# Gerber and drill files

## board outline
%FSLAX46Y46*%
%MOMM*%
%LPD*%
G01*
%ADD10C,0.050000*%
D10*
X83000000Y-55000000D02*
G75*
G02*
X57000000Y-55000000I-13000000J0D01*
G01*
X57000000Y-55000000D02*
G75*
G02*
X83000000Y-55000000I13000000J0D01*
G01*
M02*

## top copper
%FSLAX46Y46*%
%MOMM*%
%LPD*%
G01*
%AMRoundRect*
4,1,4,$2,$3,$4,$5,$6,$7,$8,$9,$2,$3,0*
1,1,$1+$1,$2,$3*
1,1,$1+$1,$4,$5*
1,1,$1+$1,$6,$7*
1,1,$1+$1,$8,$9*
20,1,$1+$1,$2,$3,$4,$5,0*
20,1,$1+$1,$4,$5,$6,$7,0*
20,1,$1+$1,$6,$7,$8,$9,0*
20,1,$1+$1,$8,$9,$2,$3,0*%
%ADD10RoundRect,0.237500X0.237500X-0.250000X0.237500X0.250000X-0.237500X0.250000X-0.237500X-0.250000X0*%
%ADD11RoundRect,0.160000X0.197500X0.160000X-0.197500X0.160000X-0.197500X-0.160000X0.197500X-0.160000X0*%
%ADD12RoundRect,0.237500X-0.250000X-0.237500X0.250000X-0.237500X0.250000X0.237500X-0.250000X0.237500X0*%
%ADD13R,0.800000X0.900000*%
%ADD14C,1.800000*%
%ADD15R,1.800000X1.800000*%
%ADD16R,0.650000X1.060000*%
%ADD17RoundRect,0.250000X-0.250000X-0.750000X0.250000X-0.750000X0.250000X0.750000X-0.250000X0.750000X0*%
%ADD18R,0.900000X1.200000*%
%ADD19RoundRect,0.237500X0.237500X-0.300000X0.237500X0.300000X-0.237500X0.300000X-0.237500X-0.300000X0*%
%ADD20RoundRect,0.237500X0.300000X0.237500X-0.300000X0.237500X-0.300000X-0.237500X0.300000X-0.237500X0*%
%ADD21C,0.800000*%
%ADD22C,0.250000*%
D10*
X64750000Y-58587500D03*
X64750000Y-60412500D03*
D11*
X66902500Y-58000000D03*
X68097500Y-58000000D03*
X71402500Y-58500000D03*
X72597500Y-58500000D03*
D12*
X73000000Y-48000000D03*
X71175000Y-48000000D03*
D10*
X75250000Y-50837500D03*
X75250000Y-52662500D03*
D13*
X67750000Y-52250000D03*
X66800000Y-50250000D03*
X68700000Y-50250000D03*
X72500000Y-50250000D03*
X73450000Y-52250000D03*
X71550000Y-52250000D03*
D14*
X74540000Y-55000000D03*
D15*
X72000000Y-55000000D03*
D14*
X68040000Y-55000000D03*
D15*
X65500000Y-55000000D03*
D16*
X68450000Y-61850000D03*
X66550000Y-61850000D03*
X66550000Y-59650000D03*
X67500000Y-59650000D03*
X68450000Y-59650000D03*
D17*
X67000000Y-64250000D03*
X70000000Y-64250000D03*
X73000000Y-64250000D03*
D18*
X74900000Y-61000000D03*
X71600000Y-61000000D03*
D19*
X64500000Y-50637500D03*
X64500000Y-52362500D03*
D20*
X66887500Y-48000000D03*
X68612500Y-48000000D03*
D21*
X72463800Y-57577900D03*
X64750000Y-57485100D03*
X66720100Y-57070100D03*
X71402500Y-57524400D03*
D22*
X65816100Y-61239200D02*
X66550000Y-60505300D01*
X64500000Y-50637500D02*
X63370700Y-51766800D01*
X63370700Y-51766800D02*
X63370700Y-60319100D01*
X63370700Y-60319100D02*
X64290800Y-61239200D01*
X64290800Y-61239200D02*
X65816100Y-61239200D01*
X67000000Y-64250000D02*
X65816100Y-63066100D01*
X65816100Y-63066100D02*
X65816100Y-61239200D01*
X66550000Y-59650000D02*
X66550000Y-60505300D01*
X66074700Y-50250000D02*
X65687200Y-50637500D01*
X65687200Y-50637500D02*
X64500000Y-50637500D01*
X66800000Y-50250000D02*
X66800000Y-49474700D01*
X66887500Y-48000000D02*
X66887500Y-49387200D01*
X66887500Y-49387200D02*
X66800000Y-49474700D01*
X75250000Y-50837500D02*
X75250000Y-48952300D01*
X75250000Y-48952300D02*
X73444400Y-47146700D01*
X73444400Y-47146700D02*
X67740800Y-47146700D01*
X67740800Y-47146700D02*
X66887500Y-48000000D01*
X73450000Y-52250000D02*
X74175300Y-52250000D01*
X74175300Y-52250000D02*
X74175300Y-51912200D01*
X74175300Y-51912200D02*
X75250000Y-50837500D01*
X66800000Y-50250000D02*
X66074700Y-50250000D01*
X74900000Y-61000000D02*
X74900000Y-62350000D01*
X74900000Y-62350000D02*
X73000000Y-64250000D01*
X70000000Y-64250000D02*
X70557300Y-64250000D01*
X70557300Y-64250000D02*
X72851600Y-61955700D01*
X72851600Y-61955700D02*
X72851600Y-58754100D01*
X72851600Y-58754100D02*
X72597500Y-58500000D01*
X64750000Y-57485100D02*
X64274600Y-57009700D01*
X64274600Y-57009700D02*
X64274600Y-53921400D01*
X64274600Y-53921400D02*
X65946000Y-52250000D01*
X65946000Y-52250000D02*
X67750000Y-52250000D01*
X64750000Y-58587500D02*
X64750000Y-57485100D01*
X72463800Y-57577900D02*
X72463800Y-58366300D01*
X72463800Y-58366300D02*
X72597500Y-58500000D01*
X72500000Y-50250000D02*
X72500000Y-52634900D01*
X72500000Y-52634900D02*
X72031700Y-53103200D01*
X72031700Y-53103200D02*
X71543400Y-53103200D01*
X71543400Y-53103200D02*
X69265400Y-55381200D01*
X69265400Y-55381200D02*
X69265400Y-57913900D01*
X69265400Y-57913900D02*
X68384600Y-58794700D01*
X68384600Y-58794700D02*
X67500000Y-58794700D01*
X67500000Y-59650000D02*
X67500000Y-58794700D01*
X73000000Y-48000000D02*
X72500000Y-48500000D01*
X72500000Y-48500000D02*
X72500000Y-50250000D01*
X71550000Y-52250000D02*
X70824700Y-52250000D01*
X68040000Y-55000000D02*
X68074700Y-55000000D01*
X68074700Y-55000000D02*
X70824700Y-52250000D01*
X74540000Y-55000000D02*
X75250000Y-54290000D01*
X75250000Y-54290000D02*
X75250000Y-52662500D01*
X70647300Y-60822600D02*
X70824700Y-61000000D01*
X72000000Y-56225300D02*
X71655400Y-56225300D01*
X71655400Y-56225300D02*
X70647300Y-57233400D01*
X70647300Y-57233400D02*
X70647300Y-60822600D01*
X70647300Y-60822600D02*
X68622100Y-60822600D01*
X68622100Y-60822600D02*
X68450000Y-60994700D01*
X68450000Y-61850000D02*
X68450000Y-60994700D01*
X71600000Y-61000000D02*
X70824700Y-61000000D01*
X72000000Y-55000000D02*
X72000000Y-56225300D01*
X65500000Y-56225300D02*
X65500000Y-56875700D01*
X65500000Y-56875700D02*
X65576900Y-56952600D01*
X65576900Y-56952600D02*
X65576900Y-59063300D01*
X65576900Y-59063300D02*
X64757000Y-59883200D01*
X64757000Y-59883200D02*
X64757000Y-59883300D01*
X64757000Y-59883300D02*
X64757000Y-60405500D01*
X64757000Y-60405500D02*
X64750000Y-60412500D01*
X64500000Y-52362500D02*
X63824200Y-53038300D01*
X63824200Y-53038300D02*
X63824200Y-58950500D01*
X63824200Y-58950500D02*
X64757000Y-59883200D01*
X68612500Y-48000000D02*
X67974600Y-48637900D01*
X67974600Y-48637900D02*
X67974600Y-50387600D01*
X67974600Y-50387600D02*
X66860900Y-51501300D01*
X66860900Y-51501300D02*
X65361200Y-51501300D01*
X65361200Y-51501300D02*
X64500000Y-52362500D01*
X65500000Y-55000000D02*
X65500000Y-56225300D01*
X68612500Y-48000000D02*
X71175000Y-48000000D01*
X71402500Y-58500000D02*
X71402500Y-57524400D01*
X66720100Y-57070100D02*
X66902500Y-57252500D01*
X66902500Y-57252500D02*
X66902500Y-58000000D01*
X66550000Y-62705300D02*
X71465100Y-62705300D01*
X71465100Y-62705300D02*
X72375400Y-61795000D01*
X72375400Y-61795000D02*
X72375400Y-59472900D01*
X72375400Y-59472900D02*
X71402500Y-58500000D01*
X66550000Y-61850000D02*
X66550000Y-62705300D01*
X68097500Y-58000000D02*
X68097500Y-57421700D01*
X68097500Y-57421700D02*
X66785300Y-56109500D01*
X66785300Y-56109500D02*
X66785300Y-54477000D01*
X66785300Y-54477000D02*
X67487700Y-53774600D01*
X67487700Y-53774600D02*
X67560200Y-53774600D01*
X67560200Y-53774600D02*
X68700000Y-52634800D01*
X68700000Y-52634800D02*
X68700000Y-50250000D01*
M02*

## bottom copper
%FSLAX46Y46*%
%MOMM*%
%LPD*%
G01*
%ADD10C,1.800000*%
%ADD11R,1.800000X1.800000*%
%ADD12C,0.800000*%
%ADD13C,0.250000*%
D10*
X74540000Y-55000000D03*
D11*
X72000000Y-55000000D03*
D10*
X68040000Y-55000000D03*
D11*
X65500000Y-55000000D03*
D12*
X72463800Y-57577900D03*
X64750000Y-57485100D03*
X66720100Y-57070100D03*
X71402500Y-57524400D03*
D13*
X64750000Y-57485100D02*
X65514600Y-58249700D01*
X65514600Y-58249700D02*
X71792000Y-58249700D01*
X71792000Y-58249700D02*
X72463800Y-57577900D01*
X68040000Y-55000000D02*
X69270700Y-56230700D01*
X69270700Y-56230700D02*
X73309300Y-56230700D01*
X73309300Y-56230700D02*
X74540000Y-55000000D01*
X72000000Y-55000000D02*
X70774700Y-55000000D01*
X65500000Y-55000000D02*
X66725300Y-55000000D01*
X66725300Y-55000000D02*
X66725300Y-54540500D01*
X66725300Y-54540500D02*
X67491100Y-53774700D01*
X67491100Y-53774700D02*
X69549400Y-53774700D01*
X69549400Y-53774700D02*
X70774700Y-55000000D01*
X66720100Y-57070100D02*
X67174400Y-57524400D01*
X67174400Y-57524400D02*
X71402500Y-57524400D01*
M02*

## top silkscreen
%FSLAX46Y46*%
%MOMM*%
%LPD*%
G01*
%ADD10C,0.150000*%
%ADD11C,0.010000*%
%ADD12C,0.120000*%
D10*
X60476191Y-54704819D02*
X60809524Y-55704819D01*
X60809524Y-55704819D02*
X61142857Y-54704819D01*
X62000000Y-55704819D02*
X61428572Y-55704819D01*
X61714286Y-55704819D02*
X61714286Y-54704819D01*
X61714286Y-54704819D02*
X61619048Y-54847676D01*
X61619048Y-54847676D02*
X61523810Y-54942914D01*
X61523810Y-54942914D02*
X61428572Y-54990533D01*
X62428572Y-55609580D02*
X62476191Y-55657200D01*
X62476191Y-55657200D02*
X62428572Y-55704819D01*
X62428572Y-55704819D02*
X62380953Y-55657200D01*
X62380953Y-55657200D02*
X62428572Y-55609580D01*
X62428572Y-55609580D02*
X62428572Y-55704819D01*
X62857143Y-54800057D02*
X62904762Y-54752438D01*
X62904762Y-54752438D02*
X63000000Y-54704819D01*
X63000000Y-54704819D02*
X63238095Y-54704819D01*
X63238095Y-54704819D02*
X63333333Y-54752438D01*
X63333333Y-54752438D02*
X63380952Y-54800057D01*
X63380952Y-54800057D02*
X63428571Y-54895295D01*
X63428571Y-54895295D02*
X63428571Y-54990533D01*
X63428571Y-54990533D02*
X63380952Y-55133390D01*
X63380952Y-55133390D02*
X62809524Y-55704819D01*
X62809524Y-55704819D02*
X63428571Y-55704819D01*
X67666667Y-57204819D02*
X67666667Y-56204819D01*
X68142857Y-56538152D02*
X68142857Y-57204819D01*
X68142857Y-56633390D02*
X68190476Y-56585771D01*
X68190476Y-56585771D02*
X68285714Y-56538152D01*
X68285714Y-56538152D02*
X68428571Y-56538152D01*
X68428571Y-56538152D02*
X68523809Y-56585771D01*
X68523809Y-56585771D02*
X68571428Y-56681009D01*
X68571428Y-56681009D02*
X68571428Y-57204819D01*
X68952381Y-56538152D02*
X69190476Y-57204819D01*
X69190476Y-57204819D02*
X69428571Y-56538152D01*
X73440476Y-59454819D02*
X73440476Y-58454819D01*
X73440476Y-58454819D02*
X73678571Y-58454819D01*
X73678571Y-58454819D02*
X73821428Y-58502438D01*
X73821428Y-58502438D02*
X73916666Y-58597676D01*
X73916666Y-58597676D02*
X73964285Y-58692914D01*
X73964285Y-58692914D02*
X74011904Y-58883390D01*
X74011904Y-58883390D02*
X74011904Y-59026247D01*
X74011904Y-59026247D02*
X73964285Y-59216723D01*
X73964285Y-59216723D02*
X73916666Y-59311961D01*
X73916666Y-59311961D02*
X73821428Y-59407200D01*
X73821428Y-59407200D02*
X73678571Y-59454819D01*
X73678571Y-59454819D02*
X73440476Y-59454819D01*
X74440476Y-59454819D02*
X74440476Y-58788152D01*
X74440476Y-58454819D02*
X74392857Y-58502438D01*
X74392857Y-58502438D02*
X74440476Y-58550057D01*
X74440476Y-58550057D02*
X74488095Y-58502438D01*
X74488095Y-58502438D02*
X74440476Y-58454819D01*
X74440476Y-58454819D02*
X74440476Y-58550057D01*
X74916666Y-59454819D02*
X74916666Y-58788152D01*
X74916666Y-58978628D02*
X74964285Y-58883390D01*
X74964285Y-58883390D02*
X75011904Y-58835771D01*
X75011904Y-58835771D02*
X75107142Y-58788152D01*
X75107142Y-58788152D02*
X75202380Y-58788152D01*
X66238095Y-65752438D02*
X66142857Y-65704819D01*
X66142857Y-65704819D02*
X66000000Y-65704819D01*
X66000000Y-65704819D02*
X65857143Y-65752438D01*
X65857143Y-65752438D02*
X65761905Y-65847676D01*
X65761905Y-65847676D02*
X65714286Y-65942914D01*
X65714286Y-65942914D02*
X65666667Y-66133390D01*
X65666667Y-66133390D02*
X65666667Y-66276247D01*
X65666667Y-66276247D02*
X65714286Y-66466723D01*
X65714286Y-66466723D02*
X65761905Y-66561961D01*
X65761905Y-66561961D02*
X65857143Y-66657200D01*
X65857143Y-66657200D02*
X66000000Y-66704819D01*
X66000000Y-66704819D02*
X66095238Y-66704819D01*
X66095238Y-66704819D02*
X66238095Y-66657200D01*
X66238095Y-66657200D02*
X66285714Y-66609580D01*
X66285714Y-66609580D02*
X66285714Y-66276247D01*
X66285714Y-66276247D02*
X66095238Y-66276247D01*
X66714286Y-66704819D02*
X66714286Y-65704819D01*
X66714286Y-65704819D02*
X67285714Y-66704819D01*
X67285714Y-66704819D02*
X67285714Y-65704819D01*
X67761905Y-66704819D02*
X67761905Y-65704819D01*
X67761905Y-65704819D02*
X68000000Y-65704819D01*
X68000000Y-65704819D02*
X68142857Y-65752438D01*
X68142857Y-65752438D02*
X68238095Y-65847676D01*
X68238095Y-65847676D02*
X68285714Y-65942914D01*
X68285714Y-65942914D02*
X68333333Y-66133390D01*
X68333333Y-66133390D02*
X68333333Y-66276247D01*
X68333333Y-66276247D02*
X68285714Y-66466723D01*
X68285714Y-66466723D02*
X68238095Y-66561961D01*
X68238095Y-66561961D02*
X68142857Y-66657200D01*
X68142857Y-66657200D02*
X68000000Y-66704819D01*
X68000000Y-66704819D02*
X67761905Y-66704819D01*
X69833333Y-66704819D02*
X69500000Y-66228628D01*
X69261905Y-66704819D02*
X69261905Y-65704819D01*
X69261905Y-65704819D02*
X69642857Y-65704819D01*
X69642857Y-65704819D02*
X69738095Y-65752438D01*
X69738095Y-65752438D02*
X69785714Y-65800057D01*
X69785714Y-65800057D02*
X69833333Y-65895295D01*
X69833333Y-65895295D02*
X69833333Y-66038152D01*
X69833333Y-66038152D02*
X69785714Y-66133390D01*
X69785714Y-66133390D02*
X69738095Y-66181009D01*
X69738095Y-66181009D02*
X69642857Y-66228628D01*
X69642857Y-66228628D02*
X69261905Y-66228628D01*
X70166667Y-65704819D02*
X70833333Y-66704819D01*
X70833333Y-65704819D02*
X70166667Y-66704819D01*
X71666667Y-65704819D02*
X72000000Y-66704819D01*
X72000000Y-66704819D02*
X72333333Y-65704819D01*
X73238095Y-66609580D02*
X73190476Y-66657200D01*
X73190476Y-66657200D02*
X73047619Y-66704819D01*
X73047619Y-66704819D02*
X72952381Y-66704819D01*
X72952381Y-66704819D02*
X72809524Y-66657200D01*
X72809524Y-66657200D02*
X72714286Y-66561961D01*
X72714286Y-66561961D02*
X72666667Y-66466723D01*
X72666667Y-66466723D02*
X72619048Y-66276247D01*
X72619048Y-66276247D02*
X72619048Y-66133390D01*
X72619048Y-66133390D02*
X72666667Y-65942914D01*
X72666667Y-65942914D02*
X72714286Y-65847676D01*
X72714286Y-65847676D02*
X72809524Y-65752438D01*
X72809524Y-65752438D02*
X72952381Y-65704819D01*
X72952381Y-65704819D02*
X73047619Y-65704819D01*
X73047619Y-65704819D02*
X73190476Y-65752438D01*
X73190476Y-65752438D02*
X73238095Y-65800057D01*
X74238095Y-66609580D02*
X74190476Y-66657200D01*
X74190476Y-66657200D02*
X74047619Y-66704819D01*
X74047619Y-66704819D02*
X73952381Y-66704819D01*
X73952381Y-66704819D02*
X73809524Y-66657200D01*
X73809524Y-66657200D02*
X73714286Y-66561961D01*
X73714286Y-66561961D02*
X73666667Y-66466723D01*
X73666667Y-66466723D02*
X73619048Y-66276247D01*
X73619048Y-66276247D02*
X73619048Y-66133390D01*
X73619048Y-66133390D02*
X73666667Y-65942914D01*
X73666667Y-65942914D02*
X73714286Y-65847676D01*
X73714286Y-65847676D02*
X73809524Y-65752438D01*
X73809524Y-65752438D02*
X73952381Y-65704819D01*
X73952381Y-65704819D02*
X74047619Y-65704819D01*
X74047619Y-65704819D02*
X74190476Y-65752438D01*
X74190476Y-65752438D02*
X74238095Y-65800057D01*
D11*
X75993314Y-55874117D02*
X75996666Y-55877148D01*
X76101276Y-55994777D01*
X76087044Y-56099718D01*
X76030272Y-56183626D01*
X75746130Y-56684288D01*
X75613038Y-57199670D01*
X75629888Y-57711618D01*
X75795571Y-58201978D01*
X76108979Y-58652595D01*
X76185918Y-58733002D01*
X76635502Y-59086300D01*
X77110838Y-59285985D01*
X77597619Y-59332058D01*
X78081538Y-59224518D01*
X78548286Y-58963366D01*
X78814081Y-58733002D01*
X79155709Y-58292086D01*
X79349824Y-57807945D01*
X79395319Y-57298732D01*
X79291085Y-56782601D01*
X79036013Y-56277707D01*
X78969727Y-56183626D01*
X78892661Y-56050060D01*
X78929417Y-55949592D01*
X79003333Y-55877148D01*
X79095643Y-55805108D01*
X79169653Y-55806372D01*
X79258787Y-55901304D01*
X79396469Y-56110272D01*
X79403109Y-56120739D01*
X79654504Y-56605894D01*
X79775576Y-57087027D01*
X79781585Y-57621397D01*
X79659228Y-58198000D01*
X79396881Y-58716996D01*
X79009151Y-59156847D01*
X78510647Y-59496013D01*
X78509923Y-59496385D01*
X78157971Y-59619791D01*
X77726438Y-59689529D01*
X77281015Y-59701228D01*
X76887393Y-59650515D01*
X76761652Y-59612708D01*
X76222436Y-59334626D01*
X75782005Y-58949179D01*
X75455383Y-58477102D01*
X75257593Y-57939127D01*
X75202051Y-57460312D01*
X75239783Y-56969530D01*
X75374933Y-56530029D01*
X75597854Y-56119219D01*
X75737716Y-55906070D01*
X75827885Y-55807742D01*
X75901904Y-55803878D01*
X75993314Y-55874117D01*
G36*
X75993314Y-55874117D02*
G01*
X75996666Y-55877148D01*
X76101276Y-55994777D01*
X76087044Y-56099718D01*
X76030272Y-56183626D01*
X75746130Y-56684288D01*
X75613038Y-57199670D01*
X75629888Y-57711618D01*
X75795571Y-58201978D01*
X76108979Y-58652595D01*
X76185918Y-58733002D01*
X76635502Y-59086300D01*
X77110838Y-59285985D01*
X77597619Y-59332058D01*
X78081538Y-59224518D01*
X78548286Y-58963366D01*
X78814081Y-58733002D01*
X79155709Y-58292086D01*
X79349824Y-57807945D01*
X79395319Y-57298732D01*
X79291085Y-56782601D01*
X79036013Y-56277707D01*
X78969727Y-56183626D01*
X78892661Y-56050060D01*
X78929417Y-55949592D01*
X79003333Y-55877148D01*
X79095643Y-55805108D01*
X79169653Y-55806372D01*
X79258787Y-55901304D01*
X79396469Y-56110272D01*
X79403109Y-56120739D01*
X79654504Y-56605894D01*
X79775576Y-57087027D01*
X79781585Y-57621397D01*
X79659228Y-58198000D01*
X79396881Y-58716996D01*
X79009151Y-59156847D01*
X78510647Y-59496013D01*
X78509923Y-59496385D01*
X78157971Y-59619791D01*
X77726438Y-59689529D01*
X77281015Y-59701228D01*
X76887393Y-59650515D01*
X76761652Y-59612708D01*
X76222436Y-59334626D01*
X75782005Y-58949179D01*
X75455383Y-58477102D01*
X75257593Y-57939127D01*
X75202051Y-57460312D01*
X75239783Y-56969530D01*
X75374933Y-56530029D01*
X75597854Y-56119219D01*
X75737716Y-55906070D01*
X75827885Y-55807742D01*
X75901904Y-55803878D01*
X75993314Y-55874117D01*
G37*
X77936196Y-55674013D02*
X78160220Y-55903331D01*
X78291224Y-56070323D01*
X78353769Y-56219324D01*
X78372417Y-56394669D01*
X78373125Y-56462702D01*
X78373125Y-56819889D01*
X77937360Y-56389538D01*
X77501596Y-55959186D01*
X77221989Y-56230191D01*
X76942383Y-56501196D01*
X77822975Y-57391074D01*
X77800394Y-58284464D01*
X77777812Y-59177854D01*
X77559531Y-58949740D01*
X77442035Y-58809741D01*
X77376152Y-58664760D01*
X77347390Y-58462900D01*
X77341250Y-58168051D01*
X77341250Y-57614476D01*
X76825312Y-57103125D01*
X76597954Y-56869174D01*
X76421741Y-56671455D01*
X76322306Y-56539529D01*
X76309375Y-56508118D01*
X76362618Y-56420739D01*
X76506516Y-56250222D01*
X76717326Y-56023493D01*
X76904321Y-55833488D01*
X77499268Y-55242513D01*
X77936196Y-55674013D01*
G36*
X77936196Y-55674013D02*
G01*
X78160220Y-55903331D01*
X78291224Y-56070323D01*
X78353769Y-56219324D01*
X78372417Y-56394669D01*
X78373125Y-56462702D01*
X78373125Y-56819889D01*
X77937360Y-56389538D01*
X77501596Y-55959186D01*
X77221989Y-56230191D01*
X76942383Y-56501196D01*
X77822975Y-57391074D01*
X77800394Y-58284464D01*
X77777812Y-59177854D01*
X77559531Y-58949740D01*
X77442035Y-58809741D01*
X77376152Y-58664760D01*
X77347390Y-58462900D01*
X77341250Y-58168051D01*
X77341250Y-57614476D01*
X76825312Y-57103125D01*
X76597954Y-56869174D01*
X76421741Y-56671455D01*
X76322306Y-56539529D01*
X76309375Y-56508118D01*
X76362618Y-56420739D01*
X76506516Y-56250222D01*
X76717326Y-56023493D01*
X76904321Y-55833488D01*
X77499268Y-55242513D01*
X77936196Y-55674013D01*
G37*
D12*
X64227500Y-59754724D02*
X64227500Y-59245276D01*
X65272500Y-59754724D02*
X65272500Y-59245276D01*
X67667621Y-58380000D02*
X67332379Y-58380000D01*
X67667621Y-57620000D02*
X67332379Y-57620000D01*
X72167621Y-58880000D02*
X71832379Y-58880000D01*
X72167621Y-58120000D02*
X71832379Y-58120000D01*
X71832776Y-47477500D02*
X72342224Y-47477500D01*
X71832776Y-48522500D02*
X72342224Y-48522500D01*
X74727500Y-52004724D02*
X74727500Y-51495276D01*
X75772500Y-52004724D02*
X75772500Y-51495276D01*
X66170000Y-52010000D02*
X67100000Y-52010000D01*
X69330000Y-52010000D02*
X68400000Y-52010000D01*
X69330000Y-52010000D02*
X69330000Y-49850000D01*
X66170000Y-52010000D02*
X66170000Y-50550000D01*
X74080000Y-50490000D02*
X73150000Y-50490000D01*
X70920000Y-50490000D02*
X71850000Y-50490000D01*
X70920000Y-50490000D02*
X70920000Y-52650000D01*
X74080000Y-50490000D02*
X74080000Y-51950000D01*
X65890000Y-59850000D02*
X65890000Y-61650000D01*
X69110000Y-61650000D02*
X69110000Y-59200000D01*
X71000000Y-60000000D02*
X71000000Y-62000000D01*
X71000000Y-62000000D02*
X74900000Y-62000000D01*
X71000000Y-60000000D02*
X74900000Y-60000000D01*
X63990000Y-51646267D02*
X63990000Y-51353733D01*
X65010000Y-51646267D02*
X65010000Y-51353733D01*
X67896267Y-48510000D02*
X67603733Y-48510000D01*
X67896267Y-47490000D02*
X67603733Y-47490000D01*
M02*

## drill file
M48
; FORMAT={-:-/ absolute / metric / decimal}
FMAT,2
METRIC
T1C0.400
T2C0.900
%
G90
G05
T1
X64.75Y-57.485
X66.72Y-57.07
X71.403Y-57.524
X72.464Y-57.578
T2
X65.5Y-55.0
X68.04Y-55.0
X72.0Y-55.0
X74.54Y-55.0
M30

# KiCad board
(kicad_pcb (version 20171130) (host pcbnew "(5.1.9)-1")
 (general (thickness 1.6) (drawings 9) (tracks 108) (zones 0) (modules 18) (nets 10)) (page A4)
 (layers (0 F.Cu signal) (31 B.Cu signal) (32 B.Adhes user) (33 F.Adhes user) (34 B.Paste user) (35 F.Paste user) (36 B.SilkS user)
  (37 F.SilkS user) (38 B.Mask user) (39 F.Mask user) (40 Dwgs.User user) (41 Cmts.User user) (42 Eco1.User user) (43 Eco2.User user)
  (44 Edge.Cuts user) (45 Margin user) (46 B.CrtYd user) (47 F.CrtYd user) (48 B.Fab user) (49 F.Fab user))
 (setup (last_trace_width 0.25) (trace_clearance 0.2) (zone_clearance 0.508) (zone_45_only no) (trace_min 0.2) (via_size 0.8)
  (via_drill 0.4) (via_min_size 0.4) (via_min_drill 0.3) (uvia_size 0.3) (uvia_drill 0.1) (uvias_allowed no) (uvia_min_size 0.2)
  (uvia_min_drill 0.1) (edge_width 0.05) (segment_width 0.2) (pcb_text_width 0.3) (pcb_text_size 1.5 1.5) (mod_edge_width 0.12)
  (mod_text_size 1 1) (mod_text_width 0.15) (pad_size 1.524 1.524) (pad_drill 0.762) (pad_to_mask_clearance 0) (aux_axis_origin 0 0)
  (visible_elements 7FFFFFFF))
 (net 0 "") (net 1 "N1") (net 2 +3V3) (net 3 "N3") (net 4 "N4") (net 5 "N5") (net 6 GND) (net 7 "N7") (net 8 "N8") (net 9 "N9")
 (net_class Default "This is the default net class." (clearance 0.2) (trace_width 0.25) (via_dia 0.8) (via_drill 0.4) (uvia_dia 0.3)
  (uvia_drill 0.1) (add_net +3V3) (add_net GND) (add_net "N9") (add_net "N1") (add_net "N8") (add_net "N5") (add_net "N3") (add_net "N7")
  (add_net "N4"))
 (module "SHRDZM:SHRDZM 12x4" (layer B.Cu) (at 70.25 49.5 180)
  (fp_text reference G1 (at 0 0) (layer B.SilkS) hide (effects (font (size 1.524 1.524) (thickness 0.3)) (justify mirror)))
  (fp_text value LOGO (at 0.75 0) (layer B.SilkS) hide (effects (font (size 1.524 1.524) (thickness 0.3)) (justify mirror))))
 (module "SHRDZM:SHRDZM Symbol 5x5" (layer F.Cu) (at 77.5 57.5)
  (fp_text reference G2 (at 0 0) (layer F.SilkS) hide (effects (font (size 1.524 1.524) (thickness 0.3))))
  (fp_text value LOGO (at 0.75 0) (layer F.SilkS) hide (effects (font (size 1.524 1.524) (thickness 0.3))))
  (fp_poly
   (pts (xy -1.506686 -1.625883) (xy -1.503334 -1.622852) (xy -1.398724 -1.505223) (xy -1.412956 -1.400282) (xy -1.469728 -1.316374)
    (xy -1.75387 -0.815712) (xy -1.886962 -0.30033) (xy -1.870112 0.211618) (xy -1.704429 0.701978) (xy -1.391021 1.152595)
    (xy -1.314082 1.233002) (xy -0.864498 1.5863) (xy -0.389162 1.785985) (xy 0.097619 1.832058) (xy 0.581538 1.724518)
    (xy 1.048286 1.463366) (xy 1.314081 1.233002) (xy 1.655709 0.792086) (xy 1.849824 0.307945) (xy 1.895319 -0.201268)
    (xy 1.791085 -0.717399) (xy 1.536013 -1.222293) (xy 1.469727 -1.316374) (xy 1.392661 -1.44994) (xy 1.429417 -1.550408)
    (xy 1.503333 -1.622852) (xy 1.595643 -1.694892) (xy 1.669653 -1.693628) (xy 1.758787 -1.598696) (xy 1.896469 -1.389728)
    (xy 1.903109 -1.379261) (xy 2.154504 -0.894106) (xy 2.275576 -0.412973) (xy 2.281585 0.121397) (xy 2.159228 0.698)
    (xy 1.896881 1.216996) (xy 1.509151 1.656847) (xy 1.010647 1.996013) (xy 1.009923 1.996385) (xy 0.657971 2.119791)
    (xy 0.226438 2.189529) (xy -0.218985 2.201228) (xy -0.612607 2.150515) (xy -0.738348 2.112708) (xy -1.277564 1.834626)
    (xy -1.717995 1.449179) (xy -2.044617 0.977102) (xy -2.242407 0.439127) (xy -2.297949 -0.039688) (xy -2.260217 -0.53047)
    (xy -2.125067 -0.969971) (xy -1.902146 -1.380781) (xy -1.762284 -1.59393) (xy -1.672115 -1.692258) (xy -1.598096 -1.696122)
    (xy -1.506686 -1.625883))
   (layer F.SilkS) (width 0.01))
  (fp_poly
   (pts (xy 0.436196 -1.825987) (xy 0.66022 -1.596669) (xy 0.791224 -1.429677) (xy 0.853769 -1.280676) (xy 0.872417 -1.105331)
    (xy 0.873125 -1.037298) (xy 0.873125 -0.680111) (xy 0.43736 -1.110462) (xy 0.001596 -1.540814) (xy -0.278011 -1.269809)
    (xy -0.557617 -0.998804) (xy 0.322975 -0.108926) (xy 0.300394 0.784464) (xy 0.277812 1.677854) (xy 0.059531 1.44974)
    (xy -0.057965 1.309741) (xy -0.123848 1.16476) (xy -0.15261 0.9629) (xy -0.15875 0.668051) (xy -0.15875 0.114476)
    (xy -0.674688 -0.396875) (xy -0.902046 -0.630826) (xy -1.078259 -0.828545) (xy -1.177694 -0.960471) (xy -1.190625 -0.991882)
    (xy -1.137382 -1.079261) (xy -0.993484 -1.249778) (xy -0.782674 -1.476507) (xy -0.595679 -1.666512) (xy -0.000732 -2.257487)
    (xy 0.436196 -1.825987))
   (layer F.SilkS) (width 0.01)))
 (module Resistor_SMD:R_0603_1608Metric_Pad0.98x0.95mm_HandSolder (layer F.Cu) (at 64.75 59.5 90)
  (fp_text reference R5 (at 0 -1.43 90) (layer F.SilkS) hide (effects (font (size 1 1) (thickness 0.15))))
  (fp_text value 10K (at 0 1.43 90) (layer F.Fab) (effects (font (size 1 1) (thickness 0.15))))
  (fp_line (start -0.254724 -0.5225) (end 0.254724 -0.5225) (layer F.SilkS) (width 0.12))
  (fp_line (start -0.254724 0.5225) (end 0.254724 0.5225) (layer F.SilkS) (width 0.12))
  (pad 2 smd roundrect (at 0.9125 0 90) (size 0.975 0.95) (layers F.Cu F.Paste F.Mask) (roundrect_rratio 0.25) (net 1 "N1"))
  (pad 1 smd roundrect (at -0.9125 0 90) (size 0.975 0.95) (layers F.Cu F.Paste F.Mask) (roundrect_rratio 0.25) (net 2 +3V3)))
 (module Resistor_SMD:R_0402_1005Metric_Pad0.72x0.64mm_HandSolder (layer F.Cu) (at 67.5 58 180)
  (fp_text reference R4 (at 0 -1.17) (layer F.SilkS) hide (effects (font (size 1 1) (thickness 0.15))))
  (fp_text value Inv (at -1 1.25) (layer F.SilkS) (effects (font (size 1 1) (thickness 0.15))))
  (fp_line (start -0.167621 -0.38) (end 0.167621 -0.38) (layer F.SilkS) (width 0.12))
  (fp_line (start -0.167621 0.38) (end 0.167621 0.38) (layer F.SilkS) (width 0.12))
  (pad 2 smd roundrect (at 0.5975 0 180) (size 0.715 0.64) (layers F.Cu F.Paste F.Mask) (roundrect_rratio 0.25) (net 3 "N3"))
  (pad 1 smd roundrect (at -0.5975 0 180) (size 0.715 0.64) (layers F.Cu F.Paste F.Mask) (roundrect_rratio 0.25) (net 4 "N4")))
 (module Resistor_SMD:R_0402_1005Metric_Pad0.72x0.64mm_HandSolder (layer F.Cu) (at 72 58.5 180)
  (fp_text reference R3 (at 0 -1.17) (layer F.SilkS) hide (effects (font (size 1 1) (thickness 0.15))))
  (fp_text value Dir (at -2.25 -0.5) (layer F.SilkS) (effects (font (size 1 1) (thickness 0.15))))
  (fp_line (start -0.167621 -0.38) (end 0.167621 -0.38) (layer F.SilkS) (width 0.12))
  (fp_line (start -0.167621 0.38) (end 0.167621 0.38) (layer F.SilkS) (width 0.12))
  (pad 2 smd roundrect (at 0.5975 0 180) (size 0.715 0.64) (layers F.Cu F.Paste F.Mask) (roundrect_rratio 0.25) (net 3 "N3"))
  (pad 1 smd roundrect (at -0.5975 0 180) (size 0.715 0.64) (layers F.Cu F.Paste F.Mask) (roundrect_rratio 0.25) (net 1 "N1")))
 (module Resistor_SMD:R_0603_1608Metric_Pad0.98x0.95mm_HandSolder (layer F.Cu) (at 72.0875 48)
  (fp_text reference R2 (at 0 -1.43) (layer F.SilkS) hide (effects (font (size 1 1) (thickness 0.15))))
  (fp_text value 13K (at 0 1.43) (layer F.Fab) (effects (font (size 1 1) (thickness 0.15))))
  (fp_line (start -0.254724 -0.5225) (end 0.254724 -0.5225) (layer F.SilkS) (width 0.12))
  (fp_line (start -0.254724 0.5225) (end 0.254724 0.5225) (layer F.SilkS) (width 0.12))
  (pad 2 smd roundrect (at 0.9125 0) (size 0.975 0.95) (layers F.Cu F.Paste F.Mask) (roundrect_rratio 0.25) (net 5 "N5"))
  (pad 1 smd roundrect (at -0.9125 0) (size 0.975 0.95) (layers F.Cu F.Paste F.Mask) (roundrect_rratio 0.25) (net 2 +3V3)))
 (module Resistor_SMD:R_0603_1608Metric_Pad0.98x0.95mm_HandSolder (layer F.Cu) (at 75.25 51.75 90)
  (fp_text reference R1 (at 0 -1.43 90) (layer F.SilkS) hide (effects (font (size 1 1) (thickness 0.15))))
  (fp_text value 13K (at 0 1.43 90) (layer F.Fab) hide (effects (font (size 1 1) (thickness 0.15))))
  (fp_line (start -0.254724 -0.5225) (end 0.254724 -0.5225) (layer F.SilkS) (width 0.12))
  (fp_line (start -0.254724 0.5225) (end 0.254724 0.5225) (layer F.SilkS) (width 0.12))
  (pad 2 smd roundrect (at 0.9125 0 90) (size 0.975 0.95) (layers F.Cu F.Paste F.Mask) (roundrect_rratio 0.25) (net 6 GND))
  (pad 1 smd roundrect (at -0.9125 0 90) (size 0.975 0.95) (layers F.Cu F.Paste F.Mask) (roundrect_rratio 0.25) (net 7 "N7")))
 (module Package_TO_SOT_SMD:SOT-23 (layer F.Cu) (at 67.75 51.25 270)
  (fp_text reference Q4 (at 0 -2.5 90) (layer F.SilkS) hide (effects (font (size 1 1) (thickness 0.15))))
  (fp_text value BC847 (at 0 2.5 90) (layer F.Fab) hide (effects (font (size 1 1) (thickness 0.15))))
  (fp_line (start 0.76 1.58) (end 0.76 0.65) (layer F.SilkS) (width 0.12))
  (fp_line (start 0.76 -1.58) (end 0.76 -0.65) (layer F.SilkS) (width 0.12))
  (fp_line (start 0.76 -1.58) (end -1.4 -1.58) (layer F.SilkS) (width 0.12))
  (fp_line (start 0.76 1.58) (end -0.7 1.58) (layer F.SilkS) (width 0.12))
  (pad 3 smd rect (at 1 0 270) (size 0.9 0.8) (layers F.Cu F.Paste F.Mask) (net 1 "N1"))
  (pad 2 smd rect (at -1 0.95 270) (size 0.9 0.8) (layers F.Cu F.Paste F.Mask) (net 6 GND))
  (pad 1 smd rect (at -1 -0.95 270) (size 0.9 0.8) (layers F.Cu F.Paste F.Mask) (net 4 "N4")))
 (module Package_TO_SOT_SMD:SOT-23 (layer F.Cu) (at 72.5 51.25 90)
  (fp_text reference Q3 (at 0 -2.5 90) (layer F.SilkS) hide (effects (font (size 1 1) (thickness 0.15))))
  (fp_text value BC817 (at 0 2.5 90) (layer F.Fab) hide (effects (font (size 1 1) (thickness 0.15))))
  (fp_line (start 0.76 1.58) (end 0.76 0.65) (layer F.SilkS) (width 0.12))
  (fp_line (start 0.76 -1.58) (end 0.76 -0.65) (layer F.SilkS) (width 0.12))
  (fp_line (start 0.76 -1.58) (end -1.4 -1.58) (layer F.SilkS) (width 0.12))
  (fp_line (start 0.76 1.58) (end -0.7 1.58) (layer F.SilkS) (width 0.12))
  (pad 3 smd rect (at 1 0 90) (size 0.9 0.8) (layers F.Cu F.Paste F.Mask) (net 5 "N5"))
  (pad 2 smd rect (at -1 0.95 90) (size 0.9 0.8) (layers F.Cu F.Paste F.Mask) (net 6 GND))
  (pad 1 smd rect (at -1 -0.95 90) (size 0.9 0.8) (layers F.Cu F.Paste F.Mask) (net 7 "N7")))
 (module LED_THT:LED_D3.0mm (layer B.Cu) (at 72 55)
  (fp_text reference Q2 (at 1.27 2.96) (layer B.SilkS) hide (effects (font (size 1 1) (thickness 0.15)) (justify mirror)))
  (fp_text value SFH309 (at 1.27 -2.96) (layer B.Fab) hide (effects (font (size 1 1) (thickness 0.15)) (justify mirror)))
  (pad 2 thru_hole circle (at 2.54 0) (size 1.8 1.8) (drill 0.9) (layers *.Cu *.Mask) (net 7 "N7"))
  (pad 1 thru_hole rect (at 0 0) (size 1.8 1.8) (drill 0.9) (layers *.Cu *.Mask) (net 2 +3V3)))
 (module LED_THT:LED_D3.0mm (layer B.Cu) (at 65.5 55)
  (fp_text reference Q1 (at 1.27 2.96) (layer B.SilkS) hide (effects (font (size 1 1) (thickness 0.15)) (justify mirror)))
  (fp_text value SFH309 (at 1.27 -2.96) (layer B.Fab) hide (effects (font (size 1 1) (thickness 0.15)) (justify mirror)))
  (pad 2 thru_hole circle (at 2.54 0) (size 1.8 1.8) (drill 0.9) (layers *.Cu *.Mask) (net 7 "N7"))
  (pad 1 thru_hole rect (at 0 0) (size 1.8 1.8) (drill 0.9) (layers *.Cu *.Mask) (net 2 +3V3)))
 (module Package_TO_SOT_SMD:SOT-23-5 (layer F.Cu) (at 67.5 60.75 270)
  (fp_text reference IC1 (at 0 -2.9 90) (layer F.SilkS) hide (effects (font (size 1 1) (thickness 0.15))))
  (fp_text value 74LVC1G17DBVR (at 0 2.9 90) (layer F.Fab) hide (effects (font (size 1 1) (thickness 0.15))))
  (fp_line (start -0.9 1.61) (end 0.9 1.61) (layer F.SilkS) (width 0.12))
  (fp_line (start 0.9 -1.61) (end -1.55 -1.61) (layer F.SilkS) (width 0.12))
  (pad 5 smd rect (at 1.1 -0.95 270) (size 1.06 0.65) (layers F.Cu F.Paste F.Mask) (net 2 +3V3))
  (pad 4 smd rect (at 1.1 0.95 270) (size 1.06 0.65) (layers F.Cu F.Paste F.Mask) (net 3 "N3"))
  (pad 3 smd rect (at -1.1 0.95 270) (size 1.06 0.65) (layers F.Cu F.Paste F.Mask) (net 6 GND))
  (pad 2 smd rect (at -1.1 0 270) (size 1.06 0.65) (layers F.Cu F.Paste F.Mask) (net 5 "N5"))
  (pad 1 smd rect (at -1.1 -0.95 270) (size 1.06 0.65) (layers F.Cu F.Paste F.Mask) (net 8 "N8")))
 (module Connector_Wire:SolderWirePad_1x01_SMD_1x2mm (layer F.Cu) (at 67 64.25)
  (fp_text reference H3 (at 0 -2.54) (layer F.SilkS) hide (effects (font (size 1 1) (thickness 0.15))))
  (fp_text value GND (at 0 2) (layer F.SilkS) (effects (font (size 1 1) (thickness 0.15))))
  (pad 1 smd roundrect (at 0 0) (size 1 2) (layers F.Cu F.Paste F.Mask) (roundrect_rratio 0.25) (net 6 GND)))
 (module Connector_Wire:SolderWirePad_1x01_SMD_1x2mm (layer F.Cu) (at 70 64.25)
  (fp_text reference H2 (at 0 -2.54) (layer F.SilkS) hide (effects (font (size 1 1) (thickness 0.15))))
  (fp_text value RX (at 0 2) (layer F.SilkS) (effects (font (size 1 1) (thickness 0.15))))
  (pad 1 smd roundrect (at 0 0) (size 1 2) (layers F.Cu F.Paste F.Mask) (roundrect_rratio 0.25) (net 1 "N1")))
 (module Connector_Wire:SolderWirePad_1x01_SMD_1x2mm (layer F.Cu) (at 73 64.25)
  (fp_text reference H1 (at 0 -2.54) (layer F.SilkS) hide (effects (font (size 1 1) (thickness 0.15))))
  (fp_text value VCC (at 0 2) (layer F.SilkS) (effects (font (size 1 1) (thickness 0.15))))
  (pad 1 smd roundrect (at 0 0) (size 1 2) (layers F.Cu F.Paste F.Mask) (roundrect_rratio 0.25) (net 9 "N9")))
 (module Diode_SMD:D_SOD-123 (layer F.Cu) (at 73.25 61)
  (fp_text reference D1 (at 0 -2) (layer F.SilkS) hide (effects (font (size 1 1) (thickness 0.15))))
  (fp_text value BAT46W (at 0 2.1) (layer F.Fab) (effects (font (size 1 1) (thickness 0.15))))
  (fp_line (start -2.25 -1) (end -2.25 1) (layer F.SilkS) (width 0.12))
  (fp_line (start -2.25 1) (end 1.65 1) (layer F.SilkS) (width 0.12))
  (fp_line (start -2.25 -1) (end 1.65 -1) (layer F.SilkS) (width 0.12))
  (pad 2 smd rect (at 1.65 0) (size 0.9 1.2) (layers F.Cu F.Paste F.Mask) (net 9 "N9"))
  (pad 1 smd rect (at -1.65 0) (size 0.9 1.2) (layers F.Cu F.Paste F.Mask) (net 2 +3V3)))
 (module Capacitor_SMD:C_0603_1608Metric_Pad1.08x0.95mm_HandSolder (layer F.Cu) (at 64.5 51.5 90)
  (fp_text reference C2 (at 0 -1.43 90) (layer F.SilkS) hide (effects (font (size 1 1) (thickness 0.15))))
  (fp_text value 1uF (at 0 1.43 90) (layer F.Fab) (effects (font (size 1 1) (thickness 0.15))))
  (fp_line (start -0.146267 -0.51) (end 0.146267 -0.51) (layer F.SilkS) (width 0.12))
  (fp_line (start -0.146267 0.51) (end 0.146267 0.51) (layer F.SilkS) (width 0.12))
  (pad 2 smd roundrect (at 0.8625 0 90) (size 1.075 0.95) (layers F.Cu F.Paste F.Mask) (roundrect_rratio 0.25) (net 6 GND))
  (pad 1 smd roundrect (at -0.8625 0 90) (size 1.075 0.95) (layers F.Cu F.Paste F.Mask) (roundrect_rratio 0.25) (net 2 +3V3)))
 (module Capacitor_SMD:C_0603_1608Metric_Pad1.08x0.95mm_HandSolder (layer F.Cu) (at 67.75 48 180)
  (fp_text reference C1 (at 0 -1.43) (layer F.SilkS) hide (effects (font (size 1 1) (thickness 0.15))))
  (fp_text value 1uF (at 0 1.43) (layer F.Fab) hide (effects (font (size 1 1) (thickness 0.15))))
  (fp_line (start -0.146267 -0.51) (end 0.146267 -0.51) (layer F.SilkS) (width 0.12))
  (fp_line (start -0.146267 0.51) (end 0.146267 0.51) (layer F.SilkS) (width 0.12))
  (pad 2 smd roundrect (at 0.8625 0 180) (size 1.075 0.95) (layers F.Cu F.Paste F.Mask) (roundrect_rratio 0.25) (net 6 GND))
  (pad 1 smd roundrect (at -0.8625 0 180) (size 1.075 0.95) (layers F.Cu F.Paste F.Mask) (roundrect_rratio 0.25) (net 2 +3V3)))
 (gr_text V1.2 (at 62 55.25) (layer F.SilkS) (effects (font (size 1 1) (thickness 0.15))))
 (gr_circle (center 70 55) (end 83 55) (layer Edge.Cuts) (width 0.05))
 (segment (start 65.8161 61.2392) (end 66.55 60.5053) (width 0.25) (layer F.Cu) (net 6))
 (segment (start 64.5 50.6375) (end 63.3707 51.7668) (width 0.25) (layer F.Cu) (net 6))
 (segment (start 63.3707 51.7668) (end 63.3707 60.3191) (width 0.25) (layer F.Cu) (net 6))
 (segment (start 63.3707 60.3191) (end 64.2908 61.2392) (width 0.25) (layer F.Cu) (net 6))
 (segment (start 64.2908 61.2392) (end 65.8161 61.2392) (width 0.25) (layer F.Cu) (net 6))
 (segment (start 67 64.25) (end 65.8161 63.0661) (width 0.25) (layer F.Cu) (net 6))
 (segment (start 65.8161 63.0661) (end 65.8161 61.2392) (width 0.25) (layer F.Cu) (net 6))
 (segment (start 66.55 59.65) (end 66.55 60.5053) (width 0.25) (layer F.Cu) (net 6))
 (segment (start 66.0747 50.25) (end 65.6872 50.6375) (width 0.25) (layer F.Cu) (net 6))
 (segment (start 65.6872 50.6375) (end 64.5 50.6375) (width 0.25) (layer F.Cu) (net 6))
 (segment (start 66.8 50.25) (end 66.8 49.4747) (width 0.25) (layer F.Cu) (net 6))
 (segment (start 66.8875 48) (end 66.8875 49.3872) (width 0.25) (layer F.Cu) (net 6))
 (segment (start 66.8875 49.3872) (end 66.8 49.4747) (width 0.25) (layer F.Cu) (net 6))
 (segment (start 75.25 50.8375) (end 75.25 48.9523) (width 0.25) (layer F.Cu) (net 6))
 (segment (start 75.25 48.9523) (end 73.4444 47.1467) (width 0.25) (layer F.Cu) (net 6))
 (segment (start 73.4444 47.1467) (end 67.7408 47.1467) (width 0.25) (layer F.Cu) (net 6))
 (segment (start 67.7408 47.1467) (end 66.8875 48) (width 0.25) (layer F.Cu) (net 6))
 (segment (start 73.45 52.25) (end 74.1753 52.25) (width 0.25) (layer F.Cu) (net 6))
 (segment (start 74.1753 52.25) (end 74.1753 51.9122) (width 0.25) (layer F.Cu) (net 6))
 (segment (start 74.1753 51.9122) (end 75.25 50.8375) (width 0.25) (layer F.Cu) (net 6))
 (segment (start 66.8 50.25) (end 66.0747 50.25) (width 0.25) (layer F.Cu) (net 6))
 (segment (start 74.9 61) (end 74.9 62.35) (width 0.25) (layer F.Cu) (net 9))
 (segment (start 74.9 62.35) (end 73 64.25) (width 0.25) (layer F.Cu) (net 9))
 (segment (start 70 64.25) (end 70.5573 64.25) (width 0.25) (layer F.Cu) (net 1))
 (segment (start 70.5573 64.25) (end 72.8516 61.9557) (width 0.25) (layer F.Cu) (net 1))
 (segment (start 72.8516 61.9557) (end 72.8516 58.7541) (width 0.25) (layer F.Cu) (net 1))
 (segment (start 72.8516 58.7541) (end 72.5975 58.5) (width 0.25) (layer F.Cu) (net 1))
 (segment (start 64.75 57.4851) (end 65.5146 58.2497) (width 0.25) (layer B.Cu) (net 1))
 (segment (start 65.5146 58.2497) (end 71.792 58.2497) (width 0.25) (layer B.Cu) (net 1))
 (segment (start 71.792 58.2497) (end 72.4638 57.5779) (width 0.25) (layer B.Cu) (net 1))
 (segment (start 64.75 57.4851) (end 64.2746 57.0097) (width 0.25) (layer F.Cu) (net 1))
 (segment (start 64.2746 57.0097) (end 64.2746 53.9214) (width 0.25) (layer F.Cu) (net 1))
 (segment (start 64.2746 53.9214) (end 65.946 52.25) (width 0.25) (layer F.Cu) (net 1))
 (segment (start 65.946 52.25) (end 67.75 52.25) (width 0.25) (layer F.Cu) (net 1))
 (segment (start 64.75 58.5875) (end 64.75 57.4851) (width 0.25) (layer F.Cu) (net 1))
 (segment (start 72.4638 57.5779) (end 72.4638 58.3663) (width 0.25) (layer F.Cu) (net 1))
 (segment (start 72.4638 58.3663) (end 72.5975 58.5) (width 0.25) (layer F.Cu) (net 1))
 (via (at 72.4638 57.5779) (size 0.8) (layers F.Cu B.Cu) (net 1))
 (via (at 64.75 57.4851) (size 0.8) (layers F.Cu B.Cu) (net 1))
 (segment (start 72.5 50.25) (end 72.5 52.6349) (width 0.25) (layer F.Cu) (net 5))
 (segment (start 72.5 52.6349) (end 72.0317 53.1032) (width 0.25) (layer F.Cu) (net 5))
 (segment (start 72.0317 53.1032) (end 71.5434 53.1032) (width 0.25) (layer F.Cu) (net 5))
 (segment (start 71.5434 53.1032) (end 69.2654 55.3812) (width 0.25) (layer F.Cu) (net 5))
 (segment (start 69.2654 55.3812) (end 69.2654 57.9139) (width 0.25) (layer F.Cu) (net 5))
 (segment (start 69.2654 57.9139) (end 68.3846 58.7947) (width 0.25) (layer F.Cu) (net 5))
 (segment (start 68.3846 58.7947) (end 67.5 58.7947) (width 0.25) (layer F.Cu) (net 5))
 (segment (start 67.5 59.65) (end 67.5 58.7947) (width 0.25) (layer F.Cu) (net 5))
 (segment (start 73 48) (end 72.5 48.5) (width 0.25) (layer F.Cu) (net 5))
 (segment (start 72.5 48.5) (end 72.5 50.25) (width 0.25) (layer F.Cu) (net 5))
 (segment (start 68.04 55) (end 69.2707 56.2307) (width 0.25) (layer B.Cu) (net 7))
 (segment (start 69.2707 56.2307) (end 73.3093 56.2307) (width 0.25) (layer B.Cu) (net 7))
 (segment (start 73.3093 56.2307) (end 74.54 55) (width 0.25) (layer B.Cu) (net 7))
 (segment (start 71.55 52.25) (end 70.8247 52.25) (width 0.25) (layer F.Cu) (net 7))
 (segment (start 68.04 55) (end 68.0747 55) (width 0.25) (layer F.Cu) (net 7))
 (segment (start 68.0747 55) (end 70.8247 52.25) (width 0.25) (layer F.Cu) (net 7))
 (segment (start 74.54 55) (end 75.25 54.29) (width 0.25) (layer F.Cu) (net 7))
 (segment (start 75.25 54.29) (end 75.25 52.6625) (width 0.25) (layer F.Cu) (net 7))
 (segment (start 70.6473 60.8226) (end 70.8247 61) (width 0.25) (layer F.Cu) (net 2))
 (segment (start 72 56.2253) (end 71.6554 56.2253) (width 0.25) (layer F.Cu) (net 2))
 (segment (start 71.6554 56.2253) (end 70.6473 57.2334) (width 0.25) (layer F.Cu) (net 2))
 (segment (start 70.6473 57.2334) (end 70.6473 60.8226) (width 0.25) (layer F.Cu) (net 2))
 (segment (start 70.6473 60.8226) (end 68.6221 60.8226) (width 0.25) (layer F.Cu) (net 2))
 (segment (start 68.6221 60.8226) (end 68.45 60.9947) (width 0.25) (layer F.Cu) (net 2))
 (segment (start 68.45 61.85) (end 68.45 60.9947) (width 0.25) (layer F.Cu) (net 2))
 (segment (start 71.6 61) (end 70.8247 61) (width 0.25) (layer F.Cu) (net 2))
 (segment (start 72 55) (end 72 56.2253) (width 0.25) (layer F.Cu) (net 2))
 (segment (start 72 55) (end 70.7747 55) (width 0.25) (layer B.Cu) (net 2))
 (segment (start 65.5 55) (end 66.7253 55) (width 0.25) (layer B.Cu) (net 2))
 (segment (start 66.7253 55) (end 66.7253 54.5405) (width 0.25) (layer B.Cu) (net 2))
 (segment (start 66.7253 54.5405) (end 67.4911 53.7747) (width 0.25) (layer B.Cu) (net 2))
 (segment (start 67.4911 53.7747) (end 69.5494 53.7747) (width 0.25) (layer B.Cu) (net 2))
 (segment (start 69.5494 53.7747) (end 70.7747 55) (width 0.25) (layer B.Cu) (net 2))
 (segment (start 65.5 56.2253) (end 65.5 56.8757) (width 0.25) (layer F.Cu) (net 2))
 (segment (start 65.5 56.8757) (end 65.5769 56.9526) (width 0.25) (layer F.Cu) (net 2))
 (segment (start 65.5769 56.9526) (end 65.5769 59.0633) (width 0.25) (layer F.Cu) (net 2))
 (segment (start 65.5769 59.0633) (end 64.757 59.8832) (width 0.25) (layer F.Cu) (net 2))
 (segment (start 64.757 59.8832) (end 64.757 59.8833) (width 0.25) (layer F.Cu) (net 2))
 (segment (start 64.757 59.8833) (end 64.757 60.4055) (width 0.25) (layer F.Cu) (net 2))
 (segment (start 64.757 60.4055) (end 64.75 60.4125) (width 0.25) (layer F.Cu) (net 2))
 (segment (start 64.5 52.3625) (end 63.8242 53.0383) (width 0.25) (layer F.Cu) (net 2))
 (segment (start 63.8242 53.0383) (end 63.8242 58.9505) (width 0.25) (layer F.Cu) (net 2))
 (segment (start 63.8242 58.9505) (end 64.757 59.8832) (width 0.25) (layer F.Cu) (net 2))
 (segment (start 68.6125 48) (end 67.9746 48.6379) (width 0.25) (layer F.Cu) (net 2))
 (segment (start 67.9746 48.6379) (end 67.9746 50.3876) (width 0.25) (layer F.Cu) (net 2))
 (segment (start 67.9746 50.3876) (end 66.8609 51.5013) (width 0.25) (layer F.Cu) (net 2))
 (segment (start 66.8609 51.5013) (end 65.3612 51.5013) (width 0.25) (layer F.Cu) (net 2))
 (segment (start 65.3612 51.5013) (end 64.5 52.3625) (width 0.25) (layer F.Cu) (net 2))
 (segment (start 65.5 55) (end 65.5 56.2253) (width 0.25) (layer F.Cu) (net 2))
 (segment (start 68.6125 48) (end 71.175 48) (width 0.25) (layer F.Cu) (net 2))
 (segment (start 71.4025 58.5) (end 71.4025 57.5244) (width 0.25) (layer F.Cu) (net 3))
 (segment (start 66.7201 57.0701) (end 67.1744 57.5244) (width 0.25) (layer B.Cu) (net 3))
 (segment (start 67.1744 57.5244) (end 71.4025 57.5244) (width 0.25) (layer B.Cu) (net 3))
 (segment (start 66.7201 57.0701) (end 66.9025 57.2525) (width 0.25) (layer F.Cu) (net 3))
 (segment (start 66.9025 57.2525) (end 66.9025 58) (width 0.25) (layer F.Cu) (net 3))
 (segment (start 66.55 62.7053) (end 71.4651 62.7053) (width 0.25) (layer F.Cu) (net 3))
 (segment (start 71.4651 62.7053) (end 72.3754 61.795) (width 0.25) (layer F.Cu) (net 3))
 (segment (start 72.3754 61.795) (end 72.3754 59.4729) (width 0.25) (layer F.Cu) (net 3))
 (segment (start 72.3754 59.4729) (end 71.4025 58.5) (width 0.25) (layer F.Cu) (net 3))
 (segment (start 66.55 61.85) (end 66.55 62.7053) (width 0.25) (layer F.Cu) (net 3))
 (via (at 66.7201 57.0701) (size 0.8) (layers F.Cu B.Cu) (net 3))
 (via (at 71.4025 57.5244) (size 0.8) (layers F.Cu B.Cu) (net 3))
 (segment (start 68.0975 58) (end 68.0975 57.4217) (width 0.25) (layer F.Cu) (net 4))
 (segment (start 68.0975 57.4217) (end 66.7853 56.1095) (width 0.25) (layer F.Cu) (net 4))
 (segment (start 66.7853 56.1095) (end 66.7853 54.477) (width 0.25) (layer F.Cu) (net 4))
 (segment (start 66.7853 54.477) (end 67.4877 53.7746) (width 0.25) (layer F.Cu) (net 4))
 (segment (start 67.4877 53.7746) (end 67.5602 53.7746) (width 0.25) (layer F.Cu) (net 4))
 (segment (start 67.5602 53.7746) (end 68.7 52.6348) (width 0.25) (layer F.Cu) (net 4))
 (segment (start 68.7 52.6348) (end 68.7 50.25) (width 0.25) (layer F.Cu) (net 4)))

